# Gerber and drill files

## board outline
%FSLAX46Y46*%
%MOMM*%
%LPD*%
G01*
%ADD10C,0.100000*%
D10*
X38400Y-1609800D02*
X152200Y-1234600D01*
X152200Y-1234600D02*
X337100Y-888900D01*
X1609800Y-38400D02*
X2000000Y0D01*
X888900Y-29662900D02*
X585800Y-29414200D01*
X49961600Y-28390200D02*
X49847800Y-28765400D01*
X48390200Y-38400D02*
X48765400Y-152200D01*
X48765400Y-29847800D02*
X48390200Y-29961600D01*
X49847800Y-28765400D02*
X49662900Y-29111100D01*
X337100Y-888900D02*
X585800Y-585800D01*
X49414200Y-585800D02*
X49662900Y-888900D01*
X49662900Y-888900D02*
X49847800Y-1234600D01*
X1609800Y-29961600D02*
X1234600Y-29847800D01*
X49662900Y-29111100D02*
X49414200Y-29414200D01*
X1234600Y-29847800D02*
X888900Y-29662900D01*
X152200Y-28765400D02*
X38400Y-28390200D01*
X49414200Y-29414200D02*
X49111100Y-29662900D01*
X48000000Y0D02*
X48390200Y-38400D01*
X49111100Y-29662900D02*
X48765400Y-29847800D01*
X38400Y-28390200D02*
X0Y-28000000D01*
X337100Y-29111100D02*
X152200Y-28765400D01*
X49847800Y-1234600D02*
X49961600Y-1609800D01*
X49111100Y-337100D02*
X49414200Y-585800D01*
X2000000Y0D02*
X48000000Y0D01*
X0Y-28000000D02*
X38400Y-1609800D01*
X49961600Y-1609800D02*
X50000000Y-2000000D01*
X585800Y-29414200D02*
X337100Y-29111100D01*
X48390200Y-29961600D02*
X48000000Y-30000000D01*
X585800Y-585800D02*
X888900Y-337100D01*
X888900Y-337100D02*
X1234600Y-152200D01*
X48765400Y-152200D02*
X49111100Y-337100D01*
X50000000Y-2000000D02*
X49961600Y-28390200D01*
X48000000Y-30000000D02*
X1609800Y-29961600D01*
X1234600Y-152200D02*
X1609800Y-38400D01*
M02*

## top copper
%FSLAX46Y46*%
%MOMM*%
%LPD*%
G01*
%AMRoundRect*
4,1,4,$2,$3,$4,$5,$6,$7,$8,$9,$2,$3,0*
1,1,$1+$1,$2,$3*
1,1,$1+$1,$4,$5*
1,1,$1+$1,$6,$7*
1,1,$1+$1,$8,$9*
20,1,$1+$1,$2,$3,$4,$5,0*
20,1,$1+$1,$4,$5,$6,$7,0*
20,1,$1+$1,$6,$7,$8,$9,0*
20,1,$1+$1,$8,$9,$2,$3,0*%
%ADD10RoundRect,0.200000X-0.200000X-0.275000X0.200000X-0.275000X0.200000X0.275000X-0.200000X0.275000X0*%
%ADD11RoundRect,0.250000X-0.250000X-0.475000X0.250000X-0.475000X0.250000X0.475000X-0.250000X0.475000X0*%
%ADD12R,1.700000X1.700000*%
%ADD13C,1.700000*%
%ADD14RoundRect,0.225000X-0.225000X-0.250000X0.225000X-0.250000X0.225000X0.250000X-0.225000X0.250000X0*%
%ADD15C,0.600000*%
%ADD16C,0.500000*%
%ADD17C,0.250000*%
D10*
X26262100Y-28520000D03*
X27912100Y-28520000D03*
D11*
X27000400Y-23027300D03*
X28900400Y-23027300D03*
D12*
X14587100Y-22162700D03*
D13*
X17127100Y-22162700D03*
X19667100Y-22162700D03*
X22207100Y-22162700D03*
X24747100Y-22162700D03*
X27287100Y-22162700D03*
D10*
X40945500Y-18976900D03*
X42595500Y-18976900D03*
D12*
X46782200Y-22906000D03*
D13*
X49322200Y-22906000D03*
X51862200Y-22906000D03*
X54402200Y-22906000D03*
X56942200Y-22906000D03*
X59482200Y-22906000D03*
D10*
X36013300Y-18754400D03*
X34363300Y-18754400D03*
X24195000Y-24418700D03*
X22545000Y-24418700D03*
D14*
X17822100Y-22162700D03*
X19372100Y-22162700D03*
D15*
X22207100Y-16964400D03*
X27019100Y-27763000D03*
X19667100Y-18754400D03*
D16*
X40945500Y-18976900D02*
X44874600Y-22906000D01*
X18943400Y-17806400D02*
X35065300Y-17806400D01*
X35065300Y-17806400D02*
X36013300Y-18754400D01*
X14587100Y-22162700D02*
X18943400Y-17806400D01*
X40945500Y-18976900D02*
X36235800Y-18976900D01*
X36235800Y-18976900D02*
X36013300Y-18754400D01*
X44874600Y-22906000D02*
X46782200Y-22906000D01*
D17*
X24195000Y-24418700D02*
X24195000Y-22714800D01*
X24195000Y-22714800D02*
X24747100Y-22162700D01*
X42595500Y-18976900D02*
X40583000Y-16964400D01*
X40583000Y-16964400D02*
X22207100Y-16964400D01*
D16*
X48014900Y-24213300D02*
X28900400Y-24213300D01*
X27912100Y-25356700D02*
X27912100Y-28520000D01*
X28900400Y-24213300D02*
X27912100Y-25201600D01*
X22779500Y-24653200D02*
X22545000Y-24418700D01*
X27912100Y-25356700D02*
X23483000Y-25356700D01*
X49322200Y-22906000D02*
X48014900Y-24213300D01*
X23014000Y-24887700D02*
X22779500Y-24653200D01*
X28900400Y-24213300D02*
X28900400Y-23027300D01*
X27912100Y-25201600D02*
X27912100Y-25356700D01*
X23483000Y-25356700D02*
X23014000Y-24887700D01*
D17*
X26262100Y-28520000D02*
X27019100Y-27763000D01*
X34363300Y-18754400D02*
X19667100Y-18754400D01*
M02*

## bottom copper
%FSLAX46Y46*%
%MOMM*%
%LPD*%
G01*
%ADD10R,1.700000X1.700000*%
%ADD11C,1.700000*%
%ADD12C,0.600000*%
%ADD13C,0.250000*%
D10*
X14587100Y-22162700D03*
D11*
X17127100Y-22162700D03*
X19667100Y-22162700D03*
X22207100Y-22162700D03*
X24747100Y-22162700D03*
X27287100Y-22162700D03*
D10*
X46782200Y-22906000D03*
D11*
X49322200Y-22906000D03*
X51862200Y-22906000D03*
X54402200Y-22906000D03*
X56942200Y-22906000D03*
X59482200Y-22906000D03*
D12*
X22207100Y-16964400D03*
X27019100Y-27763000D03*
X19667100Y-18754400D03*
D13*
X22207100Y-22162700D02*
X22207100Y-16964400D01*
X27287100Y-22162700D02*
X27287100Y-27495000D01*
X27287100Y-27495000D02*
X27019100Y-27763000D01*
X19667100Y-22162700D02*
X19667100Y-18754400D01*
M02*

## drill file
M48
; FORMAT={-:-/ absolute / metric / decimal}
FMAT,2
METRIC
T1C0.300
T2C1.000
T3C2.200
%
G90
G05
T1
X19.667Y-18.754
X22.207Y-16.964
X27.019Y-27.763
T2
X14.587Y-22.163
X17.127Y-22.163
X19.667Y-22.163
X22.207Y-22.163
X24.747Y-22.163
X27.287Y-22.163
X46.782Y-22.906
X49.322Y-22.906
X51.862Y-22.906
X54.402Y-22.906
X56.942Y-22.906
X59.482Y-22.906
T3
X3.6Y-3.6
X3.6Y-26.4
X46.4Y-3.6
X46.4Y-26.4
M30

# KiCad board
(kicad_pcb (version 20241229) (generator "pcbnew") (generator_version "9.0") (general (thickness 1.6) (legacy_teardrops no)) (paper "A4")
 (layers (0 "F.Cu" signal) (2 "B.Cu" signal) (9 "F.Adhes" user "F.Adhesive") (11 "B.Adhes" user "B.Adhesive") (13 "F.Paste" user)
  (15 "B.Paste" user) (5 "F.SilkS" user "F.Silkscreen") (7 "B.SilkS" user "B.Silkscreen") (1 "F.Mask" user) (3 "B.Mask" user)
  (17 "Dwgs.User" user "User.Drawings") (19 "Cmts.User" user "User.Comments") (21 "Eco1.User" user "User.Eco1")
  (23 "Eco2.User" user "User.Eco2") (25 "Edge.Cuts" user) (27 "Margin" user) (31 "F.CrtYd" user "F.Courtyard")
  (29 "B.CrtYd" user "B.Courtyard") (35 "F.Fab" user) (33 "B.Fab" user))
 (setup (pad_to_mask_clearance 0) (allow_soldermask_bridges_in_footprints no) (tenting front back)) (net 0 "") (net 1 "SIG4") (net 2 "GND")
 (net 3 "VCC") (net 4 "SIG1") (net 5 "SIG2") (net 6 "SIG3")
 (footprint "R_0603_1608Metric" (layer "F.Cu") (at 27.0871 28.52)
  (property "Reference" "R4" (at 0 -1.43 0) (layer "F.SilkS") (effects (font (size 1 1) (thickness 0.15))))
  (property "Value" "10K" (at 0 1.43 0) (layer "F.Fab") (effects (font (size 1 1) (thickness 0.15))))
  (pad "1" smd roundrect (at -0.825 0) (size 0.8 0.95) (layers "F.Cu" "F.Mask" "F.Paste") (roundrect_rratio 0.25) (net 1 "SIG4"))
  (pad "2" smd roundrect (at 0.825 0) (size 0.8 0.95) (layers "F.Cu" "F.Mask" "F.Paste") (roundrect_rratio 0.25) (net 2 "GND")))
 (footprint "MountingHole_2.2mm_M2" (layer "F.Cu") (at 3.6 3.6)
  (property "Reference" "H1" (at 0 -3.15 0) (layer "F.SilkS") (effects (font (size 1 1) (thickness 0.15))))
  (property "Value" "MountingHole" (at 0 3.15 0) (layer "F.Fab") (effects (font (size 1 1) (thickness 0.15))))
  (pad "" np_thru_hole circle (at 0 0) (size 2.2 2.2) (drill 2.2) (layers "*.Cu" "*.Mask")))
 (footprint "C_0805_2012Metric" (layer "F.Cu") (at 27.9504 23.0273)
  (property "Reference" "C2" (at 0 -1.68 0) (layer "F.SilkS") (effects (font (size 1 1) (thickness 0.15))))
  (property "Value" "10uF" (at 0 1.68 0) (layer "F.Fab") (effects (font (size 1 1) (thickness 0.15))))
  (pad "1" smd roundrect (at -0.95 0) (size 1 1.45) (layers "F.Cu" "F.Mask" "F.Paste") (roundrect_rratio 0.25) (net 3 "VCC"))
  (pad "2" smd roundrect (at 0.95 0) (size 1 1.45) (layers "F.Cu" "F.Mask" "F.Paste") (roundrect_rratio 0.25) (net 2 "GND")))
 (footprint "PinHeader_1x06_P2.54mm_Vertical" (layer "F.Cu") (at 14.5871 22.1627 90)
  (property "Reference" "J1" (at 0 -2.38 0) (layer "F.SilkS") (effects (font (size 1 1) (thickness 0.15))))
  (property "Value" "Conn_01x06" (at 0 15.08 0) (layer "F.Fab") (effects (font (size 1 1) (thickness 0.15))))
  (pad "1" thru_hole rect (at 0 0) (size 1.7 1.7) (drill 1) (layers "*.Cu" "*.Mask") (remove_unused_layers no) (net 3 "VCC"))
  (pad "2" thru_hole circle (at 0 2.54) (size 1.7 1.7) (drill 1) (layers "*.Cu" "*.Mask") (remove_unused_layers no) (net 2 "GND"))
  (pad "3" thru_hole circle (at 0 5.08) (size 1.7 1.7) (drill 1) (layers "*.Cu" "*.Mask") (remove_unused_layers no) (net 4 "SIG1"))
  (pad "4" thru_hole circle (at 0 7.62) (size 1.7 1.7) (drill 1) (layers "*.Cu" "*.Mask") (remove_unused_layers no) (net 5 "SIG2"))
  (pad "5" thru_hole circle (at 0 10.16) (size 1.7 1.7) (drill 1) (layers "*.Cu" "*.Mask") (remove_unused_layers no) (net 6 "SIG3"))
  (pad "6" thru_hole circle (at 0 12.7) (size 1.7 1.7) (drill 1) (layers "*.Cu" "*.Mask") (remove_unused_layers no) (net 1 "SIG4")))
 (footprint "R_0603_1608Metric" (layer "F.Cu") (at 41.7705 18.9769)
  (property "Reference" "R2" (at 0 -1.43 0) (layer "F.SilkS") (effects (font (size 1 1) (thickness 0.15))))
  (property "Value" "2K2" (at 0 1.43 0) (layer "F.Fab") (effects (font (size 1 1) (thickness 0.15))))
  (pad "1" smd roundrect (at -0.825 0) (size 0.8 0.95) (layers "F.Cu" "F.Mask" "F.Paste") (roundrect_rratio 0.25) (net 3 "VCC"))
  (pad "2" smd roundrect (at 0.825 0) (size 0.8 0.95) (layers "F.Cu" "F.Mask" "F.Paste") (roundrect_rratio 0.25) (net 5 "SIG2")))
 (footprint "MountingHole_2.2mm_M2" (layer "F.Cu") (at 46.4 26.4)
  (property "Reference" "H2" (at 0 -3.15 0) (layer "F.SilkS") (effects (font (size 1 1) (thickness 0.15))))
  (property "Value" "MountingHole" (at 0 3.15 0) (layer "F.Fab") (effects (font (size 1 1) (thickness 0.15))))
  (pad "" np_thru_hole circle (at 0 0) (size 2.2 2.2) (drill 2.2) (layers "*.Cu" "*.Mask")))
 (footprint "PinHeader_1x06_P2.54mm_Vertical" (layer "F.Cu") (at 46.7822 22.906 90)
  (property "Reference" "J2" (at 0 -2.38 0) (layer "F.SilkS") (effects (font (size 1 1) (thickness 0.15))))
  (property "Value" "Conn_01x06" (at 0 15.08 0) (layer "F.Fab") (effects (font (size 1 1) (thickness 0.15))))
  (pad "1" thru_hole rect (at 0 0) (size 1.7 1.7) (drill 1) (layers "*.Cu" "*.Mask") (remove_unused_layers no) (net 3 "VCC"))
  (pad "2" thru_hole circle (at 0 2.54) (size 1.7 1.7) (drill 1) (layers "*.Cu" "*.Mask") (remove_unused_layers no) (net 2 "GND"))
  (pad "3" thru_hole circle (at 0 5.08) (size 1.7 1.7) (drill 1) (layers "*.Cu" "*.Mask") (remove_unused_layers no) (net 4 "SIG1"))
  (pad "4" thru_hole circle (at 0 7.62) (size 1.7 1.7) (drill 1) (layers "*.Cu" "*.Mask") (remove_unused_layers no) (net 5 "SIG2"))
  (pad "5" thru_hole circle (at 0 10.16) (size 1.7 1.7) (drill 1) (layers "*.Cu" "*.Mask") (remove_unused_layers no) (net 6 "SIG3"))
  (pad "6" thru_hole circle (at 0 12.7) (size 1.7 1.7) (drill 1) (layers "*.Cu" "*.Mask") (remove_unused_layers no) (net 1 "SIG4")))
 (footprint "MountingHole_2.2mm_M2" (layer "F.Cu") (at 3.6 26.4)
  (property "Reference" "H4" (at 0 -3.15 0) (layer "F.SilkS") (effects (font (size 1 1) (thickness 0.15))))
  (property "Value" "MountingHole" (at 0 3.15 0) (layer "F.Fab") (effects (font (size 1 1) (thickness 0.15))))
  (pad "" np_thru_hole circle (at 0 0) (size 2.2 2.2) (drill 2.2) (layers "*.Cu" "*.Mask")))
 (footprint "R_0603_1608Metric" (layer "F.Cu") (at 35.1883 18.7544 180)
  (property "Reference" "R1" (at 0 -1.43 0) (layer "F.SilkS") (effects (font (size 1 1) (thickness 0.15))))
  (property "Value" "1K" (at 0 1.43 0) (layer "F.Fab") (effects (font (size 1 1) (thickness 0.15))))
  (pad "1" smd roundrect (at -0.825 0) (size 0.8 0.95) (layers "F.Cu" "F.Mask" "F.Paste") (roundrect_rratio 0.25) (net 3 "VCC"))
  (pad "2" smd roundrect (at 0.825 0) (size 0.8 0.95) (layers "F.Cu" "F.Mask" "F.Paste") (roundrect_rratio 0.25) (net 4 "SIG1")))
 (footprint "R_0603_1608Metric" (layer "F.Cu") (at 23.37 24.4187 180)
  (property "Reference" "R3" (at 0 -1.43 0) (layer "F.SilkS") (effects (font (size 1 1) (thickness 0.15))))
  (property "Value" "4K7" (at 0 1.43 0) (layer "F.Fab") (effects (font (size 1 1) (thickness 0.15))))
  (pad "1" smd roundrect (at -0.825 0) (size 0.8 0.95) (layers "F.Cu" "F.Mask" "F.Paste") (roundrect_rratio 0.25) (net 6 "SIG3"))
  (pad "2" smd roundrect (at 0.825 0) (size 0.8 0.95) (layers "F.Cu" "F.Mask" "F.Paste") (roundrect_rratio 0.25) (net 2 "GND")))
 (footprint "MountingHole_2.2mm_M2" (layer "F.Cu") (at 46.4 3.6)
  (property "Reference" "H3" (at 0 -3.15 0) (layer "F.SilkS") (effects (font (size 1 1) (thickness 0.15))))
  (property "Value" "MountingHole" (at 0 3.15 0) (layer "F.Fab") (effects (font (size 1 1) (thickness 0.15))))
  (pad "" np_thru_hole circle (at 0 0) (size 2.2 2.2) (drill 2.2) (layers "*.Cu" "*.Mask")))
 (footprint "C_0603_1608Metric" (layer "F.Cu") (at 18.5971 22.1627)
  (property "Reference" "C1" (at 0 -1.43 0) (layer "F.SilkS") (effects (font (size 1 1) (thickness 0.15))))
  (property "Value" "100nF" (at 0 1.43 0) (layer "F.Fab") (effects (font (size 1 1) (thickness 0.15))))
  (pad "1" smd roundrect (at -0.775 0) (size 0.9 0.95) (layers "F.Cu" "F.Mask" "F.Paste") (roundrect_rratio 0.25) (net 3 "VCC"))
  (pad "2" smd roundrect (at 0.775 0) (size 0.9 0.95) (layers "F.Cu" "F.Mask" "F.Paste") (roundrect_rratio 0.25) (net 2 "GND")))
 (gr_line (start 0.0384 1.6098) (end 0.1522 1.2346) (stroke (width 0.1) (type solid)) (layer "Edge.Cuts"))
 (gr_line (start 0.1522 1.2346) (end 0.3371 0.8889) (stroke (width 0.1) (type solid)) (layer "Edge.Cuts"))
 (gr_line (start 1.6098 0.0384) (end 2 0) (stroke (width 0.1) (type solid)) (layer "Edge.Cuts"))
 (gr_line (start 0.8889 29.6629) (end 0.5858 29.4142) (stroke (width 0.1) (type solid)) (layer "Edge.Cuts"))
 (gr_line (start 49.9616 28.3902) (end 49.8478 28.7654) (stroke (width 0.1) (type solid)) (layer "Edge.Cuts"))
 (gr_line (start 48.3902 0.0384) (end 48.7654 0.1522) (stroke (width 0.1) (type solid)) (layer "Edge.Cuts"))
 (gr_line (start 48.7654 29.8478) (end 48.3902 29.9616) (stroke (width 0.1) (type solid)) (layer "Edge.Cuts"))
 (gr_line (start 49.8478 28.7654) (end 49.6629 29.1111) (stroke (width 0.1) (type solid)) (layer "Edge.Cuts"))
 (gr_line (start 0.3371 0.8889) (end 0.5858 0.5858) (stroke (width 0.1) (type solid)) (layer "Edge.Cuts"))
 (gr_line (start 49.4142 0.5858) (end 49.6629 0.8889) (stroke (width 0.1) (type solid)) (layer "Edge.Cuts"))
 (gr_line (start 49.6629 0.8889) (end 49.8478 1.2346) (stroke (width 0.1) (type solid)) (layer "Edge.Cuts"))
 (gr_line (start 1.6098 29.9616) (end 1.2346 29.8478) (stroke (width 0.1) (type solid)) (layer "Edge.Cuts"))
 (gr_line (start 49.6629 29.1111) (end 49.4142 29.4142) (stroke (width 0.1) (type solid)) (layer "Edge.Cuts"))
 (gr_line (start 1.2346 29.8478) (end 0.8889 29.6629) (stroke (width 0.1) (type solid)) (layer "Edge.Cuts"))
 (gr_line (start 0.1522 28.7654) (end 0.0384 28.3902) (stroke (width 0.1) (type solid)) (layer "Edge.Cuts"))
 (gr_line (start 49.4142 29.4142) (end 49.1111 29.6629) (stroke (width 0.1) (type solid)) (layer "Edge.Cuts"))
 (gr_line (start 48 0) (end 48.3902 0.0384) (stroke (width 0.1) (type solid)) (layer "Edge.Cuts"))
 (gr_line (start 49.1111 29.6629) (end 48.7654 29.8478) (stroke (width 0.1) (type solid)) (layer "Edge.Cuts"))
 (gr_line (start 0.0384 28.3902) (end 0 28) (stroke (width 0.1) (type solid)) (layer "Edge.Cuts"))
 (gr_line (start 0.3371 29.1111) (end 0.1522 28.7654) (stroke (width 0.1) (type solid)) (layer "Edge.Cuts"))
 (gr_line (start 49.8478 1.2346) (end 49.9616 1.6098) (stroke (width 0.1) (type solid)) (layer "Edge.Cuts"))
 (gr_line (start 49.1111 0.3371) (end 49.4142 0.5858) (stroke (width 0.1) (type solid)) (layer "Edge.Cuts"))
 (gr_line (start 2 0) (end 48 0) (stroke (width 0.1) (type solid)) (layer "Edge.Cuts"))
 (gr_line (start 0 28) (end 0.0384 1.6098) (stroke (width 0.1) (type solid)) (layer "Edge.Cuts"))
 (gr_line (start 49.9616 1.6098) (end 50 2) (stroke (width 0.1) (type solid)) (layer "Edge.Cuts"))
 (gr_line (start 0.5858 29.4142) (end 0.3371 29.1111) (stroke (width 0.1) (type solid)) (layer "Edge.Cuts"))
 (gr_line (start 48.3902 29.9616) (end 48 30) (stroke (width 0.1) (type solid)) (layer "Edge.Cuts"))
 (gr_line (start 0.5858 0.5858) (end 0.8889 0.3371) (stroke (width 0.1) (type solid)) (layer "Edge.Cuts"))
 (gr_line (start 0.8889 0.3371) (end 1.2346 0.1522) (stroke (width 0.1) (type solid)) (layer "Edge.Cuts"))
 (gr_line (start 48.7654 0.1522) (end 49.1111 0.3371) (stroke (width 0.1) (type solid)) (layer "Edge.Cuts"))
 (gr_line (start 50 2) (end 49.9616 28.3902) (stroke (width 0.1) (type solid)) (layer "Edge.Cuts"))
 (gr_line (start 48 30) (end 1.6098 29.9616) (stroke (width 0.1) (type solid)) (layer "Edge.Cuts"))
 (gr_line (start 1.2346 0.1522) (end 1.6098 0.0384) (stroke (width 0.1) (type solid)) (layer "Edge.Cuts"))
 (segment (start 40.9455 18.9769) (end 44.8746 22.906) (width 0.5) (layer "F.Cu") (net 3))
 (segment (start 18.9434 17.8064) (end 35.0653 17.8064) (width 0.5) (layer "F.Cu") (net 3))
 (segment (start 35.0653 17.8064) (end 36.0133 18.7544) (width 0.5) (layer "F.Cu") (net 3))
 (segment (start 14.5871 22.1627) (end 18.9434 17.8064) (width 0.5) (layer "F.Cu") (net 3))
 (segment (start 40.9455 18.9769) (end 36.2358 18.9769) (width 0.5) (layer "F.Cu") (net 3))
 (segment (start 36.2358 18.9769) (end 36.0133 18.7544) (width 0.5) (layer "F.Cu") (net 3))
 (segment (start 44.8746 22.906) (end 46.7822 22.906) (width 0.5) (layer "F.Cu") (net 3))
 (segment (start 24.195 24.4187) (end 24.195 22.7148) (width 0.25) (layer "F.Cu") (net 6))
 (segment (start 24.195 22.7148) (end 24.7471 22.1627) (width 0.25) (layer "F.Cu") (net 6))
 (segment (start 42.5955 18.9769) (end 40.583 16.9644) (width 0.25) (layer "F.Cu") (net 5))
 (segment (start 40.583 16.9644) (end 22.2071 16.9644) (width 0.25) (layer "F.Cu") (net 5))
 (via (at 22.2071 16.9644) (size 0.6) (drill 0.3) (layers "F.Cu" "B.Cu") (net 5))
 (segment (start 22.2071 22.1627) (end 22.2071 16.9644) (width 0.25) (layer "B.Cu") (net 5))
 (segment (start 48.0149 24.2133) (end 28.9004 24.2133) (width 0.5) (layer "F.Cu") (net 2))
 (segment (start 27.9121 25.3567) (end 27.9121 28.52) (width 0.5) (layer "F.Cu") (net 2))
 (segment (start 28.9004 24.2133) (end 27.9121 25.2016) (width 0.5) (layer "F.Cu") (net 2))
 (segment (start 22.7795 24.6532) (end 22.545 24.4187) (width 0.5) (layer "F.Cu") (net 2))
 (segment (start 27.9121 25.3567) (end 23.483 25.3567) (width 0.5) (layer "F.Cu") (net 2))
 (segment (start 49.3222 22.906) (end 48.0149 24.2133) (width 0.5) (layer "F.Cu") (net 2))
 (segment (start 23.014 24.8877) (end 22.7795 24.6532) (width 0.5) (layer "F.Cu") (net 2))
 (segment (start 28.9004 24.2133) (end 28.9004 23.0273) (width 0.5) (layer "F.Cu") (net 2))
 (segment (start 27.9121 25.2016) (end 27.9121 25.3567) (width 0.5) (layer "F.Cu") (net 2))
 (segment (start 23.483 25.3567) (end 23.014 24.8877) (width 0.5) (layer "F.Cu") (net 2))
 (segment (start 26.2621 28.52) (end 27.0191 27.763) (width 0.25) (layer "F.Cu") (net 1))
 (via (at 27.0191 27.763) (size 0.6) (drill 0.3) (layers "F.Cu" "B.Cu") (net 1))
 (segment (start 27.2871 22.1627) (end 27.2871 27.495) (width 0.25) (layer "B.Cu") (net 1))
 (segment (start 27.2871 27.495) (end 27.0191 27.763) (width 0.25) (layer "B.Cu") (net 1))
 (segment (start 34.3633 18.7544) (end 19.6671 18.7544) (width 0.25) (layer "F.Cu") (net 4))
 (via (at 19.6671 18.7544) (size 0.6) (drill 0.3) (layers "F.Cu" "B.Cu") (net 4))
 (segment (start 19.6671 22.1627) (end 19.6671 18.7544) (width 0.25) (layer "B.Cu") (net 4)))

